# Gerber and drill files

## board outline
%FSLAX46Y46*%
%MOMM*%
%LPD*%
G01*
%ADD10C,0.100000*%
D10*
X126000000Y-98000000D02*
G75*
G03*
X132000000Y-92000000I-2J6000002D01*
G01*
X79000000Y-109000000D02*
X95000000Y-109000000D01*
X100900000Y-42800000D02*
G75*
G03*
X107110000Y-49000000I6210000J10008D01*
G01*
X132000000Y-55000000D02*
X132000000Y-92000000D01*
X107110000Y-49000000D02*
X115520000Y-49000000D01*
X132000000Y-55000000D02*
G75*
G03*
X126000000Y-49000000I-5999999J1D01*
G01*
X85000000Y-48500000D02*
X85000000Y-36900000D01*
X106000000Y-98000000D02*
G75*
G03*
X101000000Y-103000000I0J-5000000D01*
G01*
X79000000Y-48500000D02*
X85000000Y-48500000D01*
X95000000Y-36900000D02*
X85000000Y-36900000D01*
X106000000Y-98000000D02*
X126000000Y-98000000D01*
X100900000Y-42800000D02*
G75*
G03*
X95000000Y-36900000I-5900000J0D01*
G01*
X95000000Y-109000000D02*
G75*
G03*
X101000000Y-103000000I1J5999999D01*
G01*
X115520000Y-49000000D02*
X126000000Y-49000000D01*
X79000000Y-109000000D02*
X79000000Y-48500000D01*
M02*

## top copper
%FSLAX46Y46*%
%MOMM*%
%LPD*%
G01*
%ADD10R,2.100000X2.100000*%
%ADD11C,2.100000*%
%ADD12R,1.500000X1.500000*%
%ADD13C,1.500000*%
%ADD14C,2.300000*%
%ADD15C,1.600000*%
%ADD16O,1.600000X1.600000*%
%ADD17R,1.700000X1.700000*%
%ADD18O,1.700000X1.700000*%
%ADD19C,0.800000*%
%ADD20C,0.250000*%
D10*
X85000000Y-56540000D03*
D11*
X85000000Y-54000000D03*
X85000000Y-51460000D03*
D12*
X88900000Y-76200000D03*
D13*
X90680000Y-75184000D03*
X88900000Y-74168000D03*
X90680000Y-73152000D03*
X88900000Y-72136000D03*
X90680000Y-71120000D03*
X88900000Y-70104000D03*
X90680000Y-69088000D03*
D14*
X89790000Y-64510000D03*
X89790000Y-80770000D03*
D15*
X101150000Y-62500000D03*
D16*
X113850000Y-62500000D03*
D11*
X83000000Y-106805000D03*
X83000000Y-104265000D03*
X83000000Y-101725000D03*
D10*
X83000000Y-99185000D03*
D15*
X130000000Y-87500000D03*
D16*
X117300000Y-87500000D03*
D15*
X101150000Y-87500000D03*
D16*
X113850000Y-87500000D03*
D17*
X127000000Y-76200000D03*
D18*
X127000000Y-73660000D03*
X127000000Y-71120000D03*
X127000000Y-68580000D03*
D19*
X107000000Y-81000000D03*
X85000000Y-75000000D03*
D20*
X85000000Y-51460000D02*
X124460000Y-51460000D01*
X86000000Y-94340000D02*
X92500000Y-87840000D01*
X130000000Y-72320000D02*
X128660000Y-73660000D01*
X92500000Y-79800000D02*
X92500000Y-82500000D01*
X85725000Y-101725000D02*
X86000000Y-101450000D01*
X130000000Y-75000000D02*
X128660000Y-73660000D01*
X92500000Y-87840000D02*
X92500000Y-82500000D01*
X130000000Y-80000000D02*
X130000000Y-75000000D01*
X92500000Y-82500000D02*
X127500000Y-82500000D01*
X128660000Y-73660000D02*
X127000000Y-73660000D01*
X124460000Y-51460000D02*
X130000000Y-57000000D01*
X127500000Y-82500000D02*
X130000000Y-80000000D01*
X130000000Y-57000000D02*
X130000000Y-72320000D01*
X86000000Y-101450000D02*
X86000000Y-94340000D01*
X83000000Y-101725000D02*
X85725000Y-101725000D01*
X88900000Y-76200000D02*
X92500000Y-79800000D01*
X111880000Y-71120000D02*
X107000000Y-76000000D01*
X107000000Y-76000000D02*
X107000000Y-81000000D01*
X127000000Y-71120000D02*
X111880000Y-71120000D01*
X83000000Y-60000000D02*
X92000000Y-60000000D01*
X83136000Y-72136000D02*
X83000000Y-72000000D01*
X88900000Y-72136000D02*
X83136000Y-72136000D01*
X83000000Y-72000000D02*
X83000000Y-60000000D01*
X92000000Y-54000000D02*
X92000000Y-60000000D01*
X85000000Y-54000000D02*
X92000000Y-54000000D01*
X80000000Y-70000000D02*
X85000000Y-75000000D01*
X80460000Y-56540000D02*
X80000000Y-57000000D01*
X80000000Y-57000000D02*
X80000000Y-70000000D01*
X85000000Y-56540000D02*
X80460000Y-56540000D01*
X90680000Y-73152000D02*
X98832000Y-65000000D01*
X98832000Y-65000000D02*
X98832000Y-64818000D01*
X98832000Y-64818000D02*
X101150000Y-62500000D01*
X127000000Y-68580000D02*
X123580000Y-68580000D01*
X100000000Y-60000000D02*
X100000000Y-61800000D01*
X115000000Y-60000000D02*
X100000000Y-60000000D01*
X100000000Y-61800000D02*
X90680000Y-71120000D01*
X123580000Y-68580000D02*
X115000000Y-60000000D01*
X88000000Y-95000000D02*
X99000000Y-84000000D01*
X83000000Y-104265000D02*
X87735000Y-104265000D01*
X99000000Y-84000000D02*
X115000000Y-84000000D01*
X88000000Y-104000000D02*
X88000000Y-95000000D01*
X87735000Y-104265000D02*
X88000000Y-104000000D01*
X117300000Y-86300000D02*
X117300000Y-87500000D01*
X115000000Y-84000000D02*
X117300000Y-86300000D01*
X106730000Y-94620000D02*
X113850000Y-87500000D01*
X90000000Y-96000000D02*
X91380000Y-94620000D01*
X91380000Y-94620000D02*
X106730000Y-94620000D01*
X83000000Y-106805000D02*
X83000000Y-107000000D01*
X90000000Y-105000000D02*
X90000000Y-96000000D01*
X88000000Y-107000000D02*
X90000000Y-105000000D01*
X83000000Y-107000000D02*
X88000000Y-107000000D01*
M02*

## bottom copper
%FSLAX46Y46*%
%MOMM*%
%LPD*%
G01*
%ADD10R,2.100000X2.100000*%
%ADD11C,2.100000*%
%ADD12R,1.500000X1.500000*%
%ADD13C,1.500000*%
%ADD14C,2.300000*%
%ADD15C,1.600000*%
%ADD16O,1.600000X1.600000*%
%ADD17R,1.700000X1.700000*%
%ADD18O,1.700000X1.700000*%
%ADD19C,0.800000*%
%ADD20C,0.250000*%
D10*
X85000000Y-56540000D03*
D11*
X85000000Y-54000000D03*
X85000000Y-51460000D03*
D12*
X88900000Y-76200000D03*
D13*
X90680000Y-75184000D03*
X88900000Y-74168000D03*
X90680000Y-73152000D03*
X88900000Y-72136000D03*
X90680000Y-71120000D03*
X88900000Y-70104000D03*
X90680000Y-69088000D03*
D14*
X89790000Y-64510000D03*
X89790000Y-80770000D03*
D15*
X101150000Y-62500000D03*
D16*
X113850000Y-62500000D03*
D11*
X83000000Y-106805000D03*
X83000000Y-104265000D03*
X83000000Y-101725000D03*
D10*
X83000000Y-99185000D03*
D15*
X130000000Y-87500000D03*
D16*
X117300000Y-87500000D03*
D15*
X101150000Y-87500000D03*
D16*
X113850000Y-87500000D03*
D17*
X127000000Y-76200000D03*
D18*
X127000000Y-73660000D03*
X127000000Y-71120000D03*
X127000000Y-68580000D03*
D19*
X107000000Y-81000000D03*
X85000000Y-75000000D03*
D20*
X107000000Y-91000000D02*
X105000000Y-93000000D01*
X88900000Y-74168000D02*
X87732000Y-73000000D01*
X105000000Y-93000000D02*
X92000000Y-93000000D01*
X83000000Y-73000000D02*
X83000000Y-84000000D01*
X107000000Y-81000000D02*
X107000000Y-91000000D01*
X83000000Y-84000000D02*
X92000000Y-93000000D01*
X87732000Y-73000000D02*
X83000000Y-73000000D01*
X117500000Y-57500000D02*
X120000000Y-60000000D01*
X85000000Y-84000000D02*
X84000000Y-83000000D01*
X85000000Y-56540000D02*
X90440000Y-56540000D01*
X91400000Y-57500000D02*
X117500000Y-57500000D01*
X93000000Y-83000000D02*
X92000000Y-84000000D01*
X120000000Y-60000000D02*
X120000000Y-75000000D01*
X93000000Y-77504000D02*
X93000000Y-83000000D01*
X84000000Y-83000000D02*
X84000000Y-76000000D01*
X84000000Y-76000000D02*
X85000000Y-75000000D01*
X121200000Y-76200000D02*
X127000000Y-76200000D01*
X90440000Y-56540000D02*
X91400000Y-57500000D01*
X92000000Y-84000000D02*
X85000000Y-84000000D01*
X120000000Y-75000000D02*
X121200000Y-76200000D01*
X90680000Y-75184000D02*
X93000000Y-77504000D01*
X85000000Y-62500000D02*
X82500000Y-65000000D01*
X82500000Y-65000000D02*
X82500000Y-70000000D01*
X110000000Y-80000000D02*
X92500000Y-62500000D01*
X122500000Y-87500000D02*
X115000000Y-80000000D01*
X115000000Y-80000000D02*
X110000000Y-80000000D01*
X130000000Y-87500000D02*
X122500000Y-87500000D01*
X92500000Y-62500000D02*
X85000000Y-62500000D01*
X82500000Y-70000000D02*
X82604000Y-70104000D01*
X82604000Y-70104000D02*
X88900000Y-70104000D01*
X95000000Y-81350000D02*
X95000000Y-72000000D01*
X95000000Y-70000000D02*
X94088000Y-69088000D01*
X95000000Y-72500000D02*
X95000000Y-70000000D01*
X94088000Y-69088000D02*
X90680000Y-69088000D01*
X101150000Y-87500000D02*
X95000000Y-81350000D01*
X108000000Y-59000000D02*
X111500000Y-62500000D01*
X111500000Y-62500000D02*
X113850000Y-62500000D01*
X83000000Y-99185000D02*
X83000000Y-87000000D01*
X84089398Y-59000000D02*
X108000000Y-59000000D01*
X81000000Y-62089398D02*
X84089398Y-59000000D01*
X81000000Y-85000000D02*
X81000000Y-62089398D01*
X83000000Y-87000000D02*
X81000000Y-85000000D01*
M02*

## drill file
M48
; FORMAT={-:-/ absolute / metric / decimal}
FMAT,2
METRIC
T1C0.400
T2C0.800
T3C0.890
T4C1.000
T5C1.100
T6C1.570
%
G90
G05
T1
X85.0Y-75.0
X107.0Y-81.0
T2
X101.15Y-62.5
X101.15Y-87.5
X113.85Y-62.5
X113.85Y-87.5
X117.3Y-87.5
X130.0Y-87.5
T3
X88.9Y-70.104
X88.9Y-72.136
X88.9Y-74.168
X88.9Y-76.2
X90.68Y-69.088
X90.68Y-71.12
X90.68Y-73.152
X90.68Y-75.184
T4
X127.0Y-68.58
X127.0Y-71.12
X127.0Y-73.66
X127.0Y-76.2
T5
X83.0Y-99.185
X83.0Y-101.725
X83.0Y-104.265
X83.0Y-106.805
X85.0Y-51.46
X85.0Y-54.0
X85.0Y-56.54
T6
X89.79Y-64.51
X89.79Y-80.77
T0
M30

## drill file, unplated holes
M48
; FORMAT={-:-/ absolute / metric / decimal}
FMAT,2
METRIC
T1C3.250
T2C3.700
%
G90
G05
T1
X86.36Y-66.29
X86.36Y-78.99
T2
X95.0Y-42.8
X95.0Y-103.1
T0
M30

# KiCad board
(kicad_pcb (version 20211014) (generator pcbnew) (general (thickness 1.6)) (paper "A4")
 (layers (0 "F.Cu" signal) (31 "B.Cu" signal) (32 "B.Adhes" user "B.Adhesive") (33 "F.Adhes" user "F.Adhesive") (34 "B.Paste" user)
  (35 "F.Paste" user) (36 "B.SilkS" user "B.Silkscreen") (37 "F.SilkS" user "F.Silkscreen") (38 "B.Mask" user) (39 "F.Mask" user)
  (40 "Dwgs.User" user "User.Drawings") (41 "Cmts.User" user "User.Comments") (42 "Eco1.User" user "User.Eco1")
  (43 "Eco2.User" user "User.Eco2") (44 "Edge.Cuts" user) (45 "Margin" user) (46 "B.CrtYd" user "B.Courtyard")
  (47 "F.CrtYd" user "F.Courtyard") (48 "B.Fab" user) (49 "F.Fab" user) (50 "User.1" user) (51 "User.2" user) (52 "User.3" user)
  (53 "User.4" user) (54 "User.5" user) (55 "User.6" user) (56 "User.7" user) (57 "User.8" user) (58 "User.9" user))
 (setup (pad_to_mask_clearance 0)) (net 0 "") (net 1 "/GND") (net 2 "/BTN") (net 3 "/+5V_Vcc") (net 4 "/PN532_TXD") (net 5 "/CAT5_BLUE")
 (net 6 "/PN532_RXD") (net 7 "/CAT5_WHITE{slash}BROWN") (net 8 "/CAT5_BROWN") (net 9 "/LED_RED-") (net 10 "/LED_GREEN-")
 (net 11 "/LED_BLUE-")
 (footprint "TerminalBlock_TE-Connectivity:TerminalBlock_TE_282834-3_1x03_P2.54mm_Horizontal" (layer "F.Cu") (at 85 56.54 90)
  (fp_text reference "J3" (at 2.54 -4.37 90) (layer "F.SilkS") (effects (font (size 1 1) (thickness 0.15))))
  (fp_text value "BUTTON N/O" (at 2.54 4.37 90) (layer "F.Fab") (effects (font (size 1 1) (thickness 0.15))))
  (pad "1" thru_hole rect locked (at 0 0 90) (size 2.1 2.1) (drill 1.1) (layers *.Cu *.Mask) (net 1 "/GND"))
  (pad "2" thru_hole circle locked (at 2.54 0 90) (size 2.1 2.1) (drill 1.1) (layers *.Cu *.Mask) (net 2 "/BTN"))
  (pad "3" thru_hole circle locked (at 5.08 0 90) (size 2.1 2.1) (drill 1.1) (layers *.Cu *.Mask) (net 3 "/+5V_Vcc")))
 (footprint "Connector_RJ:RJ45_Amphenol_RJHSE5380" (layer "F.Cu") (at 88.9 76.2 90)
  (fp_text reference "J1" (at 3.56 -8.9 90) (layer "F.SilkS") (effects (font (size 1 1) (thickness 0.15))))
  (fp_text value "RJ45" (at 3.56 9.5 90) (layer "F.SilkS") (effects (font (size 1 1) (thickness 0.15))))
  (pad "" np_thru_hole circle locked (at -2.79 -2.54 90) (size 3.25 3.25) (drill 3.25) (layers *.Cu *.Mask))
  (pad "" np_thru_hole circle locked (at 9.91 -2.54 90) (size 3.25 3.25) (drill 3.25) (layers *.Cu *.Mask))
  (pad "1" thru_hole rect locked (at 0 0 90) (size 1.5 1.5) (drill 0.89) (layers *.Cu *.Mask) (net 3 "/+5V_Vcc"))
  (pad "2" thru_hole circle locked (at 1.016 1.78 90) (size 1.5 1.5) (drill 0.89) (layers *.Cu *.Mask) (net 1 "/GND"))
  (pad "3" thru_hole circle locked (at 2.032 0 90) (size 1.5 1.5) (drill 0.89) (layers *.Cu *.Mask) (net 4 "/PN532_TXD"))
  (pad "4" thru_hole circle locked (at 3.048 1.78 90) (size 1.5 1.5) (drill 0.89) (layers *.Cu *.Mask) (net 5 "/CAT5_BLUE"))
  (pad "5" thru_hole circle locked (at 4.064 0 90) (size 1.5 1.5) (drill 0.89) (layers *.Cu *.Mask) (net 2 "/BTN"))
  (pad "6" thru_hole circle locked (at 5.08 1.78 90) (size 1.5 1.5) (drill 0.89) (layers *.Cu *.Mask) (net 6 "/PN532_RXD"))
  (pad "7" thru_hole circle locked (at 6.096 0 90) (size 1.5 1.5) (drill 0.89) (layers *.Cu *.Mask) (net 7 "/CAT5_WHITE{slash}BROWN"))
  (pad "8" thru_hole circle locked (at 7.112 1.78 90) (size 1.5 1.5) (drill 0.89) (layers *.Cu *.Mask) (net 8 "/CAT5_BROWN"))
  (pad "SH" thru_hole circle locked (at 11.69 0.89 90) (size 2.3 2.3) (drill 1.57) (layers *.Cu *.Mask))
  (pad "SH" thru_hole circle locked (at -4.57 0.89 90) (size 2.3 2.3) (drill 1.57) (layers *.Cu *.Mask)))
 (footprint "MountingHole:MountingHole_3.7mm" (layer "F.Cu") (at 95 42.8)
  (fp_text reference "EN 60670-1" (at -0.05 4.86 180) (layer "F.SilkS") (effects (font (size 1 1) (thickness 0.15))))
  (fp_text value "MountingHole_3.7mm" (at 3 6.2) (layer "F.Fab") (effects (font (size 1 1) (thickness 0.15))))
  (pad "" np_thru_hole circle locked (at 0 0) (size 3.7 3.7) (drill 3.7) (layers *.Cu *.Mask)))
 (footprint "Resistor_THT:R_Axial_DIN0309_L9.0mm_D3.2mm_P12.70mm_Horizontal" (layer "F.Cu") (at 101.15 62.5)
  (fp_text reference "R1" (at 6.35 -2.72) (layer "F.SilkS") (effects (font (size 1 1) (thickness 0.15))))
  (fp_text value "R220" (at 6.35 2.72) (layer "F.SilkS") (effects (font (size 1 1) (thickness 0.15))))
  (pad "1" thru_hole circle locked (at 0 0) (size 1.6 1.6) (drill 0.8) (layers *.Cu *.Mask) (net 5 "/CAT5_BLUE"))
  (pad "2" thru_hole oval locked (at 12.7 0) (size 1.6 1.6) (drill 0.8) (layers *.Cu *.Mask) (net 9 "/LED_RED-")))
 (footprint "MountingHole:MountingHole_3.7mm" (layer "F.Cu") (at 95 103.1)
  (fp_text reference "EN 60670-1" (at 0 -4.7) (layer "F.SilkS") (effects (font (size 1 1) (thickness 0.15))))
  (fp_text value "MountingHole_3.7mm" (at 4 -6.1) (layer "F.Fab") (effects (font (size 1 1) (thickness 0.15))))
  (pad "" np_thru_hole circle locked (at 0 0) (size 3.7 3.7) (drill 3.7) (layers *.Cu *.Mask)))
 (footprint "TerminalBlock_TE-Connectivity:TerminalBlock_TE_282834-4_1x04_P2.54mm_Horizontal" (layer "F.Cu") (at 83 99.185 -90)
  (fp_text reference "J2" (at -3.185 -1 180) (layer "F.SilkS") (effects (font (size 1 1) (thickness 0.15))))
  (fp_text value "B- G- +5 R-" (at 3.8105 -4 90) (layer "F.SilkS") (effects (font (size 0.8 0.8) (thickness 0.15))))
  (pad "1" thru_hole rect locked (at 0 0 270) (size 2.1 2.1) (drill 1.1) (layers *.Cu *.Mask) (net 9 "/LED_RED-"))
  (pad "2" thru_hole circle locked (at 2.54 0 270) (size 2.1 2.1) (drill 1.1) (layers *.Cu *.Mask) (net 3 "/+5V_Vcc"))
  (pad "3" thru_hole circle locked (at 5.08 0 270) (size 2.1 2.1) (drill 1.1) (layers *.Cu *.Mask) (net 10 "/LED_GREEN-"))
  (pad "4" thru_hole circle locked (at 7.62 0 270) (size 2.1 2.1) (drill 1.1) (layers *.Cu *.Mask) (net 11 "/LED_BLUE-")))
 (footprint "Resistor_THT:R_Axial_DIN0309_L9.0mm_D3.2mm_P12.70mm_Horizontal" (layer "F.Cu") (at 130 87.5 180)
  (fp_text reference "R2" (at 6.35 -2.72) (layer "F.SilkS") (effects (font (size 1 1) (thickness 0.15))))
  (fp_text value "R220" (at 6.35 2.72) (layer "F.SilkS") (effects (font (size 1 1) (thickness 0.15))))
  (pad "1" thru_hole circle locked (at 0 0 180) (size 1.6 1.6) (drill 0.8) (layers *.Cu *.Mask) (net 7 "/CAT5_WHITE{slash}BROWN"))
  (pad "2" thru_hole oval locked (at 12.7 0 180) (size 1.6 1.6) (drill 0.8) (layers *.Cu *.Mask) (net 10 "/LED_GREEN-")))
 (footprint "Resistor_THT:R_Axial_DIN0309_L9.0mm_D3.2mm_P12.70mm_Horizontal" (layer "F.Cu") (at 101.15 87.5)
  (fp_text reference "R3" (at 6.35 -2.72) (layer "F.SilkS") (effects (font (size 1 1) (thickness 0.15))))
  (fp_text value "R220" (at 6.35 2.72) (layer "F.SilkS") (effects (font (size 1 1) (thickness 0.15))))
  (pad "1" thru_hole circle locked (at 0 0) (size 1.6 1.6) (drill 0.8) (layers *.Cu *.Mask) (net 8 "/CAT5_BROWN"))
  (pad "2" thru_hole oval locked (at 12.7 0) (size 1.6 1.6) (drill 0.8) (layers *.Cu *.Mask) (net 11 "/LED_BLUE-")))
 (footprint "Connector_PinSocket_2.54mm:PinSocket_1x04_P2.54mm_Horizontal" (layer "B.Cu") (at 127 76.2)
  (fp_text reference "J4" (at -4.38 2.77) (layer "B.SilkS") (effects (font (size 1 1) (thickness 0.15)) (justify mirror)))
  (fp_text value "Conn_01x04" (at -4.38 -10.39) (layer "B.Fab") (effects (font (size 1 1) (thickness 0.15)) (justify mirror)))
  (pad "1" thru_hole rect locked (at 0 0) (size 1.7 1.7) (drill 1) (layers *.Cu *.Mask) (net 1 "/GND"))
  (pad "2" thru_hole oval locked (at 0 -2.54) (size 1.7 1.7) (drill 1) (layers *.Cu *.Mask) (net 3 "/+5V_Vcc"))
  (pad "3" thru_hole oval locked (at 0 -5.08) (size 1.7 1.7) (drill 1) (layers *.Cu *.Mask) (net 4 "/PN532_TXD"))
  (pad "4" thru_hole oval locked (at 0 -7.62) (size 1.7 1.7) (drill 1) (layers *.Cu *.Mask) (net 6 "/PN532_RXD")))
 (gr_arc (start 132 92) (mid 130.24264 96.24264) (end 126 98) (layer "Edge.Cuts") (width 0.1))
 (gr_line (start 79 109) (end 95 109) (layer "Edge.Cuts") (width 0.1))
 (gr_arc (start 107.11 49) (mid 102.722401 47.184668) (end 100.9 42.8) (layer "Edge.Cuts") (width 0.1))
 (gr_line (start 132 55) (end 132 92) (layer "Edge.Cuts") (width 0.1))
 (gr_line (start 107.11 49) (end 115.52 49) (layer "Edge.Cuts") (width 0.1))
 (gr_arc (start 126 49) (mid 130.242641 50.757359) (end 132 55) (layer "Edge.Cuts") (width 0.1))
 (gr_line (start 85 48.5) (end 85 36.9) (layer "Edge.Cuts") (width 0.1))
 (gr_arc (start 101 103) (mid 102.464466 99.464466) (end 106 98) (layer "Edge.Cuts") (width 0.1))
 (gr_line (start 79 48.5) (end 85 48.5) (layer "Edge.Cuts") (width 0.1))
 (gr_line (start 95 36.9) (end 85 36.9) (layer "Edge.Cuts") (width 0.1))
 (gr_line (start 106 98) (end 126 98) (layer "Edge.Cuts") (width 0.1))
 (gr_arc (start 95 36.9) (mid 99.17193 38.62807) (end 100.9 42.8) (layer "Edge.Cuts") (width 0.1))
 (gr_arc (start 101 103) (mid 99.242641 107.242641) (end 95 109) (layer "Edge.Cuts") (width 0.1))
 (gr_line (start 115.52 49) (end 126 49) (layer "Edge.Cuts") (width 0.1))
 (gr_line (start 79 109) (end 79 48.5) (layer "Edge.Cuts") (width 0.1))
 (segment (start 85 51.46) (end 124.46 51.46) (width 0.25) (layer "F.Cu") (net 3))
 (segment (start 86 94.34) (end 92.5 87.84) (width 0.25) (layer "F.Cu") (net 3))
 (segment (start 130 72.32) (end 128.66 73.66) (width 0.25) (layer "F.Cu") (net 3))
 (segment (start 92.5 79.8) (end 92.5 82.5) (width 0.25) (layer "F.Cu") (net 3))
 (segment (start 85.725 101.725) (end 86 101.45) (width 0.25) (layer "F.Cu") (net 3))
 (segment (start 130 75) (end 128.66 73.66) (width 0.25) (layer "F.Cu") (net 3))
 (segment (start 92.5 87.84) (end 92.5 82.5) (width 0.25) (layer "F.Cu") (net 3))
 (segment (start 130 80) (end 130 75) (width 0.25) (layer "F.Cu") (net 3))
 (segment (start 92.5 82.5) (end 127.5 82.5) (width 0.25) (layer "F.Cu") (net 3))
 (segment (start 128.66 73.66) (end 127 73.66) (width 0.25) (layer "F.Cu") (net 3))
 (segment (start 124.46 51.46) (end 130 57) (width 0.25) (layer "F.Cu") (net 3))
 (segment (start 127.5 82.5) (end 130 80) (width 0.25) (layer "F.Cu") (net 3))
 (segment (start 130 57) (end 130 72.32) (width 0.25) (layer "F.Cu") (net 3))
 (segment (start 86 101.45) (end 86 94.34) (width 0.25) (layer "F.Cu") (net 3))
 (segment (start 83 101.725) (end 85.725 101.725) (width 0.25) (layer "F.Cu") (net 3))
 (segment (start 88.9 76.2) (end 92.5 79.8) (width 0.25) (layer "F.Cu") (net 3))
 (segment (start 111.88 71.12) (end 107 76) (width 0.25) (layer "F.Cu") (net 4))
 (segment (start 107 76) (end 107 81) (width 0.25) (layer "F.Cu") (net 4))
 (segment (start 127 71.12) (end 111.88 71.12) (width 0.25) (layer "F.Cu") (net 4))
 (via (at 107 81) (size 0.8) (drill 0.4) (layers "F.Cu" "B.Cu") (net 4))
 (segment (start 107 91) (end 105 93) (width 0.25) (layer "B.Cu") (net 4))
 (segment (start 88.9 74.168) (end 87.732 73) (width 0.25) (layer "B.Cu") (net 4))
 (segment (start 105 93) (end 92 93) (width 0.25) (layer "B.Cu") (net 4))
 (segment (start 83 73) (end 83 84) (width 0.25) (layer "B.Cu") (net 4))
 (segment (start 107 81) (end 107 91) (width 0.25) (layer "B.Cu") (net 4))
 (segment (start 83 84) (end 92 93) (width 0.25) (layer "B.Cu") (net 4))
 (segment (start 87.732 73) (end 83 73) (width 0.25) (layer "B.Cu") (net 4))
 (segment (start 83 60) (end 92 60) (width 0.25) (layer "F.Cu") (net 2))
 (segment (start 83.136 72.136) (end 83 72) (width 0.25) (layer "F.Cu") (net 2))
 (segment (start 88.9 72.136) (end 83.136 72.136) (width 0.25) (layer "F.Cu") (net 2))
 (segment (start 83 72) (end 83 60) (width 0.25) (layer "F.Cu") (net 2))
 (segment (start 92 54) (end 92 60) (width 0.25) (layer "F.Cu") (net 2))
 (segment (start 85 54) (end 92 54) (width 0.25) (layer "F.Cu") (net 2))
 (segment (start 80 70) (end 85 75) (width 0.25) (layer "F.Cu") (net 1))
 (segment (start 80.46 56.54) (end 80 57) (width 0.25) (layer "F.Cu") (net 1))
 (segment (start 80 57) (end 80 70) (width 0.25) (layer "F.Cu") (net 1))
 (segment (start 85 56.54) (end 80.46 56.54) (width 0.25) (layer "F.Cu") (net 1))
 (via (at 85 75) (size 0.8) (drill 0.4) (layers "F.Cu" "B.Cu") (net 1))
 (segment (start 117.5 57.5) (end 120 60) (width 0.25) (layer "B.Cu") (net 1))
 (segment (start 85 84) (end 84 83) (width 0.25) (layer "B.Cu") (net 1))
 (segment (start 85 56.54) (end 90.44 56.54) (width 0.25) (layer "B.Cu") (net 1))
 (segment (start 91.4 57.5) (end 117.5 57.5) (width 0.25) (layer "B.Cu") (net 1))
 (segment (start 93 83) (end 92 84) (width 0.25) (layer "B.Cu") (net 1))
 (segment (start 120 60) (end 120 75) (width 0.25) (layer "B.Cu") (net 1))
 (segment (start 93 77.504) (end 93 83) (width 0.25) (layer "B.Cu") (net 1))
 (segment (start 84 83) (end 84 76) (width 0.25) (layer "B.Cu") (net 1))
 (segment (start 84 76) (end 85 75) (width 0.25) (layer "B.Cu") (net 1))
 (segment (start 121.2 76.2) (end 127 76.2) (width 0.25) (layer "B.Cu") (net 1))
 (segment (start 90.44 56.54) (end 91.4 57.5) (width 0.25) (layer "B.Cu") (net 1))
 (segment (start 92 84) (end 85 84) (width 0.25) (layer "B.Cu") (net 1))
 (segment (start 120 75) (end 121.2 76.2) (width 0.25) (layer "B.Cu") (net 1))
 (segment (start 90.68 75.184) (end 93 77.504) (width 0.25) (layer "B.Cu") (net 1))
 (segment (start 85 62.5) (end 82.5 65) (width 0.25) (layer "B.Cu") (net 7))
 (segment (start 82.5 65) (end 82.5 70) (width 0.25) (layer "B.Cu") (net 7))
 (segment (start 110 80) (end 92.5 62.5) (width 0.25) (layer "B.Cu") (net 7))
 (segment (start 122.5 87.5) (end 115 80) (width 0.25) (layer "B.Cu") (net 7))
 (segment (start 115 80) (end 110 80) (width 0.25) (layer "B.Cu") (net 7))
 (segment (start 130 87.5) (end 122.5 87.5) (width 0.25) (layer "B.Cu") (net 7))
 (segment (start 92.5 62.5) (end 85 62.5) (width 0.25) (layer "B.Cu") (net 7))
 (segment (start 82.5 70) (end 82.604 70.104) (width 0.25) (layer "B.Cu") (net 7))
 (segment (start 82.604 70.104) (end 88.9 70.104) (width 0.25) (layer "B.Cu") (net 7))
 (segment (start 90.68 73.152) (end 98.832 65) (width 0.25) (layer "F.Cu") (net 5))
 (segment (start 98.832 65) (end 98.832 64.818) (width 0.25) (layer "F.Cu") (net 5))
 (segment (start 98.832 64.818) (end 101.15 62.5) (width 0.25) (layer "F.Cu") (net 5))
 (segment (start 127 68.58) (end 123.58 68.58) (width 0.25) (layer "F.Cu") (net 6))
 (segment (start 100 60) (end 100 61.8) (width 0.25) (layer "F.Cu") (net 6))
 (segment (start 115 60) (end 100 60) (width 0.25) (layer "F.Cu") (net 6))
 (segment (start 100 61.8) (end 90.68 71.12) (width 0.25) (layer "F.Cu") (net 6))
 (segment (start 123.58 68.58) (end 115 60) (width 0.25) (layer "F.Cu") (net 6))
 (segment (start 95 81.35) (end 95 72) (width 0.25) (layer "B.Cu") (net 8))
 (segment (start 95 70) (end 94.088 69.088) (width 0.25) (layer "B.Cu") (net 8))
 (segment (start 95 72.5) (end 95 70) (width 0.25) (layer "B.Cu") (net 8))
 (segment (start 94.088 69.088) (end 90.68 69.088) (width 0.25) (layer "B.Cu") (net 8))
 (segment (start 101.15 87.5) (end 95 81.35) (width 0.25) (layer "B.Cu") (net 8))
 (segment (start 108 59) (end 111.5 62.5) (width 0.25) (layer "B.Cu") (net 9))
 (segment (start 111.5 62.5) (end 113.85 62.5) (width 0.25) (layer "B.Cu") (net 9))
 (segment (start 83 99.185) (end 83 87) (width 0.25) (layer "B.Cu") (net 9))
 (segment (start 84.089398 59) (end 108 59) (width 0.25) (layer "B.Cu") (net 9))
 (segment (start 81 62.089398) (end 84.089398 59) (width 0.25) (layer "B.Cu") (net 9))
 (segment (start 81 85) (end 81 62.089398) (width 0.25) (layer "B.Cu") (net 9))
 (segment (start 83 87) (end 81 85) (width 0.25) (layer "B.Cu") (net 9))
 (segment (start 88 95) (end 99 84) (width 0.25) (layer "F.Cu") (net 10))
 (segment (start 83 104.265) (end 87.735 104.265) (width 0.25) (layer "F.Cu") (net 10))
 (segment (start 99 84) (end 115 84) (width 0.25) (layer "F.Cu") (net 10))
 (segment (start 88 104) (end 88 95) (width 0.25) (layer "F.Cu") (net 10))
 (segment (start 87.735 104.265) (end 88 104) (width 0.25) (layer "F.Cu") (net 10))
 (segment (start 117.3 86.3) (end 117.3 87.5) (width 0.25) (layer "F.Cu") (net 10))
 (segment (start 115 84) (end 117.3 86.3) (width 0.25) (layer "F.Cu") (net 10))
 (segment (start 106.73 94.62) (end 113.85 87.5) (width 0.25) (layer "F.Cu") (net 11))
 (segment (start 90 96) (end 91.38 94.62) (width 0.25) (layer "F.Cu") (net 11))
 (segment (start 91.38 94.62) (end 106.73 94.62) (width 0.25) (layer "F.Cu") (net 11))
 (segment (start 83 106.805) (end 83 107) (width 0.25) (layer "F.Cu") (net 11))
 (segment (start 90 105) (end 90 96) (width 0.25) (layer "F.Cu") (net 11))
 (segment (start 88 107) (end 90 105) (width 0.25) (layer "F.Cu") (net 11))
 (segment (start 83 107) (end 88 107) (width 0.25) (layer "F.Cu") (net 11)))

